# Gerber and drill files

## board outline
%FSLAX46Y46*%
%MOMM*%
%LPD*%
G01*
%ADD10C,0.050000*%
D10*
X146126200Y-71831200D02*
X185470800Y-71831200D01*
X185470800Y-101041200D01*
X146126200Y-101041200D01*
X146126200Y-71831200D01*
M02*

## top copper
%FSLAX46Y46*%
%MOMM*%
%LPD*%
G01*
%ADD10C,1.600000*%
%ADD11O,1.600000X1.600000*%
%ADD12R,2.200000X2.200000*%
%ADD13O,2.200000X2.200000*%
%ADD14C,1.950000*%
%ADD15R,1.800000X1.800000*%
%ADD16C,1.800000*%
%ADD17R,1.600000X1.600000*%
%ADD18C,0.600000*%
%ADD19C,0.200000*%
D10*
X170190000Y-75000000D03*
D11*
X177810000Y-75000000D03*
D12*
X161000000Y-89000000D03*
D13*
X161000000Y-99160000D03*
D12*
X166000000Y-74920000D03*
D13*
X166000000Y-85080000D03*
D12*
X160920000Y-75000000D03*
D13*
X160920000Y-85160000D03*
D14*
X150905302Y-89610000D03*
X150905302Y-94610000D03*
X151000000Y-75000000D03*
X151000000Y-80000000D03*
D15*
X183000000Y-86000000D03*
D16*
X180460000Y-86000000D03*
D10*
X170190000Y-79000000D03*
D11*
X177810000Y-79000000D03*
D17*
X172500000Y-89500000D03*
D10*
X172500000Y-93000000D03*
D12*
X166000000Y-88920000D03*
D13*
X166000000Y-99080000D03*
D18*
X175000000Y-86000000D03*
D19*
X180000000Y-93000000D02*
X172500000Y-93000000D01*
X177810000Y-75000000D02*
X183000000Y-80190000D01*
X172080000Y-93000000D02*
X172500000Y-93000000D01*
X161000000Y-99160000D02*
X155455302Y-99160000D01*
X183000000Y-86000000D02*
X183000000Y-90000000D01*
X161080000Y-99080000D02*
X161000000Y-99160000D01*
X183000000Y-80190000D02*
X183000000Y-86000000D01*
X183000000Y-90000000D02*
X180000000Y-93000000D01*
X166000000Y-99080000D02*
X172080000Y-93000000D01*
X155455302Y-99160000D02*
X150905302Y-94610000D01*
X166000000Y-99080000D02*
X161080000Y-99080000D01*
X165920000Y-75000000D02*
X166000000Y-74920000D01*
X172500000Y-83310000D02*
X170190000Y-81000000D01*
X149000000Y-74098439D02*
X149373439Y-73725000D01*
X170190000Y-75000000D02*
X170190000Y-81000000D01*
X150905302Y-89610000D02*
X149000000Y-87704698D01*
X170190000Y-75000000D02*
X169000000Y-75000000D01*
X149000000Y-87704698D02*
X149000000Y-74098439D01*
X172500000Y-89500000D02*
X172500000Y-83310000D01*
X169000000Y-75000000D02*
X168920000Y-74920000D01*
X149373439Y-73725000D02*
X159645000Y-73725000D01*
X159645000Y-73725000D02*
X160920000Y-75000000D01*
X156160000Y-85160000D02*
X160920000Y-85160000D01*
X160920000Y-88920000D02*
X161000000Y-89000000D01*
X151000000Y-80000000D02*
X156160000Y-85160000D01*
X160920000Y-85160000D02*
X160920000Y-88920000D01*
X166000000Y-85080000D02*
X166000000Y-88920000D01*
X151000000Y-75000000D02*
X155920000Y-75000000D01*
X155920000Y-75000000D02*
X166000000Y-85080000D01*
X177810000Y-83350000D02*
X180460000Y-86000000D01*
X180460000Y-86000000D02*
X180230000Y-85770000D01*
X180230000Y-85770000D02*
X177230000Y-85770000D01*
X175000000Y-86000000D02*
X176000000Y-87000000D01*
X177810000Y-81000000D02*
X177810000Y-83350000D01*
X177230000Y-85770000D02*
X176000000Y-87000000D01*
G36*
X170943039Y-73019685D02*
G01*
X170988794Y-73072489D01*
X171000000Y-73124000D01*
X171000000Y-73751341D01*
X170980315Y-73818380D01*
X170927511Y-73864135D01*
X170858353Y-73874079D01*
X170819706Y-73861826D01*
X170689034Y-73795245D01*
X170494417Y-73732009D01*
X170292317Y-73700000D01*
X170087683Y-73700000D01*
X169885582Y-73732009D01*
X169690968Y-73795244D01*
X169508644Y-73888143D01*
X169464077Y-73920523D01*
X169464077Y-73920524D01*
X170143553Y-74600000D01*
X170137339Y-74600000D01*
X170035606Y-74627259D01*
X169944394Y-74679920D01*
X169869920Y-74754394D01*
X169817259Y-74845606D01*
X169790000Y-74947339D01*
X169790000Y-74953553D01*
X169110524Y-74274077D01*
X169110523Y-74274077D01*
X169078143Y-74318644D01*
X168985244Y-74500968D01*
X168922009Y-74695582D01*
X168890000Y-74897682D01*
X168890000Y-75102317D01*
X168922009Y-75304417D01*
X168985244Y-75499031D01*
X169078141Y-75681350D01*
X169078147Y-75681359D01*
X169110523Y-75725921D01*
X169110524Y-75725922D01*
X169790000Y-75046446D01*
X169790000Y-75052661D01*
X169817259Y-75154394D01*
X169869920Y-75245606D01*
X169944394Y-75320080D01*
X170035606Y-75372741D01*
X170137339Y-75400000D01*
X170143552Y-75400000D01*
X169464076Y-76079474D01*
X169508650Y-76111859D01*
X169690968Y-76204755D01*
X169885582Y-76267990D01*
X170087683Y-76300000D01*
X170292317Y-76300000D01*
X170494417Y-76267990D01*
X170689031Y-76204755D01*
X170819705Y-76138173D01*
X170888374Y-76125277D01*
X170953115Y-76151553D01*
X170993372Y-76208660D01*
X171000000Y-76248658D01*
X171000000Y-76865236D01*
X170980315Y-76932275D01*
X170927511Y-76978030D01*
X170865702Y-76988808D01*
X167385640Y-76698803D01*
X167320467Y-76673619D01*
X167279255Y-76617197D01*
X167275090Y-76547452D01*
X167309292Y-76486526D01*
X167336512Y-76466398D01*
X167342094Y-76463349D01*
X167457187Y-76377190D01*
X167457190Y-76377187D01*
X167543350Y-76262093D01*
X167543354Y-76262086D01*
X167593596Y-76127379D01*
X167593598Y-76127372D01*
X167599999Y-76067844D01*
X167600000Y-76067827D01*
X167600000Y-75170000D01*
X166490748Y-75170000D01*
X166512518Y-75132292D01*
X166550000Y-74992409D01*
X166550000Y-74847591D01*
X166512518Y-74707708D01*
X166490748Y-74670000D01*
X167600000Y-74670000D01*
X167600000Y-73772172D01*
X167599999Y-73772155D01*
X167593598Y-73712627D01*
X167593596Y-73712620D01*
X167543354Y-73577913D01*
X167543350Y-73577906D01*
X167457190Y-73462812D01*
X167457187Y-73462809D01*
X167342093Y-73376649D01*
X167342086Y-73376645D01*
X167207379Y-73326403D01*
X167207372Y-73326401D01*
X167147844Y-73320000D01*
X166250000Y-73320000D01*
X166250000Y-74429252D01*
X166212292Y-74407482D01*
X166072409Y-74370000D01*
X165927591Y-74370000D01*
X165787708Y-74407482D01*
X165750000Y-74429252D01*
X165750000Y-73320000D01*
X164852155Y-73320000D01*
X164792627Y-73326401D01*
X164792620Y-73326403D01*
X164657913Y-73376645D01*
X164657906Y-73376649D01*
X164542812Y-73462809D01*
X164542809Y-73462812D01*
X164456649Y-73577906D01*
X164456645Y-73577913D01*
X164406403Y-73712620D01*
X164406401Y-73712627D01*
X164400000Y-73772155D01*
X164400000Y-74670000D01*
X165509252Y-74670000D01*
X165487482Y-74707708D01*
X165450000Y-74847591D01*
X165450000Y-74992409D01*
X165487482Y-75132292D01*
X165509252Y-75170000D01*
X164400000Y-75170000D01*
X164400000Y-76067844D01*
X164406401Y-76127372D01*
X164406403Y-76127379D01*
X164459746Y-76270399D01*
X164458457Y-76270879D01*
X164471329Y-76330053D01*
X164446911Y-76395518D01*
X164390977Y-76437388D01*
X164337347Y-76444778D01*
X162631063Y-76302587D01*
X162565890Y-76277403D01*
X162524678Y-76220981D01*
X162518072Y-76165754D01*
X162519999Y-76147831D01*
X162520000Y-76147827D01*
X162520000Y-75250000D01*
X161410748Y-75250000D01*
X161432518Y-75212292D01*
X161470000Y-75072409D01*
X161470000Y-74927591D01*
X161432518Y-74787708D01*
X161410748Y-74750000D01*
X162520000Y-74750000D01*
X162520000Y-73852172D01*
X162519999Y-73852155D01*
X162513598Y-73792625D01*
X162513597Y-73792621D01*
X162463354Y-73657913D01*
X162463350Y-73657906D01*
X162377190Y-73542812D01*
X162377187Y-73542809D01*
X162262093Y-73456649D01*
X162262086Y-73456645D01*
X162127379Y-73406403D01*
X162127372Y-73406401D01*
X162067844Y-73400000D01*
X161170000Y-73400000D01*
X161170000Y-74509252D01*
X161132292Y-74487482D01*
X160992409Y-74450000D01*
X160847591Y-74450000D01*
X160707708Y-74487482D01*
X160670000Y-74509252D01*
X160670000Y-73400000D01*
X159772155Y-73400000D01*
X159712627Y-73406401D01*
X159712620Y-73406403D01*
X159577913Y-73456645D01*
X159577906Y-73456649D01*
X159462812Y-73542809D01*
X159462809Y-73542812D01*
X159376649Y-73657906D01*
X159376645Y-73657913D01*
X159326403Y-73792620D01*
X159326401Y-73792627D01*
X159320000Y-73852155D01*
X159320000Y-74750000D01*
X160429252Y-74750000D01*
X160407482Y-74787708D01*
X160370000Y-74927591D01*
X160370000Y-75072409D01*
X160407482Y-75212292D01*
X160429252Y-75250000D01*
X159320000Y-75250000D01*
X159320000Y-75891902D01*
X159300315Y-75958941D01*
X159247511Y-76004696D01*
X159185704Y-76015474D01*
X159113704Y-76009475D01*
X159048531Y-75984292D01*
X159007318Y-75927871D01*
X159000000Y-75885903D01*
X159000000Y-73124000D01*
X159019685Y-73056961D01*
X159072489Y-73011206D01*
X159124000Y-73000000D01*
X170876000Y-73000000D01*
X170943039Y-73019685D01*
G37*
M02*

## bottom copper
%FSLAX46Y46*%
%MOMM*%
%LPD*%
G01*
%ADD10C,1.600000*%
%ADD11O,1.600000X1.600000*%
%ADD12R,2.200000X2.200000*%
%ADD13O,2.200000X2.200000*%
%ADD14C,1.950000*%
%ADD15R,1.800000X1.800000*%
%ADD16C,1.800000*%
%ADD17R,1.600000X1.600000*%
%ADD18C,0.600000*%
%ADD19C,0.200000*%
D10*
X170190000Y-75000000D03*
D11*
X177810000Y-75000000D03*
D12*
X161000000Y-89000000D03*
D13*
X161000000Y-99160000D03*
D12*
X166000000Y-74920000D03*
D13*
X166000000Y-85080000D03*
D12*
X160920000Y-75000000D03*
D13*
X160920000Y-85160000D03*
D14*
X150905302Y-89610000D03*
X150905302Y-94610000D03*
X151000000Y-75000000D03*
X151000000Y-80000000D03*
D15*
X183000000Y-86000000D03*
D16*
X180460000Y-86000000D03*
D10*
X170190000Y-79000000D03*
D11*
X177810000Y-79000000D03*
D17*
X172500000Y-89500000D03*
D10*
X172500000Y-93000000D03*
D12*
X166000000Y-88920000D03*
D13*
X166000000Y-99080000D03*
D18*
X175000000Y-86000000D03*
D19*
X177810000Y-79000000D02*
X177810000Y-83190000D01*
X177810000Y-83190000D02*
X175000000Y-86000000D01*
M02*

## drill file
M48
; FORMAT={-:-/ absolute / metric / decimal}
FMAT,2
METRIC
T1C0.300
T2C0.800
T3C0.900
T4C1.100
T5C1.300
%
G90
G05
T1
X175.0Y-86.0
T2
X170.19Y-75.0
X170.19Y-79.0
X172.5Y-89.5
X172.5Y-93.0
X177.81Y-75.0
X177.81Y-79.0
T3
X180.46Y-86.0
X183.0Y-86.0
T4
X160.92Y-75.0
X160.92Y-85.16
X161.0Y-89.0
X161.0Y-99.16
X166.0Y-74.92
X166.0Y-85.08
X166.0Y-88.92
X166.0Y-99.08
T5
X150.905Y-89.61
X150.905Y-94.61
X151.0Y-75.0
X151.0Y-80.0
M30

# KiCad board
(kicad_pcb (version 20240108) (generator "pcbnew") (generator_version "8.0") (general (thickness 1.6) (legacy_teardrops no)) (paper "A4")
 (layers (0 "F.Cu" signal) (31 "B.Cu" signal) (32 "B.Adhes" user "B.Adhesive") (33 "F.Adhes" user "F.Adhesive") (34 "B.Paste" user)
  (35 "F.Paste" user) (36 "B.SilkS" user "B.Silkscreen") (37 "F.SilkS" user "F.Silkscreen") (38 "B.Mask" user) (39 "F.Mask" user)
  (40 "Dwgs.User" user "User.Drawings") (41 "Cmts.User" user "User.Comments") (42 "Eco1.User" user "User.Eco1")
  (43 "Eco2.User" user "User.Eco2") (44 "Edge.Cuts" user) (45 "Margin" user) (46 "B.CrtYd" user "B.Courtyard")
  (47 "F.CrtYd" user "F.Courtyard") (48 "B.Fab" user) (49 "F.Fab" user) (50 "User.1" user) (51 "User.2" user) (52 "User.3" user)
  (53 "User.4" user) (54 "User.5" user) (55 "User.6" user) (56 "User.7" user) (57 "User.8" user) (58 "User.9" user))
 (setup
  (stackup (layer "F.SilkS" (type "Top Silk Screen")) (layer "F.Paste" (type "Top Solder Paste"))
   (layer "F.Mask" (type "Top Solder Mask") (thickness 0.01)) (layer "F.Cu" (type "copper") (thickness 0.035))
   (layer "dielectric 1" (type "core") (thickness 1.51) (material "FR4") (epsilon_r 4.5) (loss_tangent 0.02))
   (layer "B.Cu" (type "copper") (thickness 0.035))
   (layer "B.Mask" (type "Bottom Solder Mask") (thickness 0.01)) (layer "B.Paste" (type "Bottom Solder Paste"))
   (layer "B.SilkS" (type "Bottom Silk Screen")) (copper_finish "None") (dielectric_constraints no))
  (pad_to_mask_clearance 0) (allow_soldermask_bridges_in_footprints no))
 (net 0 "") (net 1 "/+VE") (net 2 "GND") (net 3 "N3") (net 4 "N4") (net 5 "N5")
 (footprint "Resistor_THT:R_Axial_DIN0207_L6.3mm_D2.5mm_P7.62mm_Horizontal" (layer "F.Cu") (at 170.19 75)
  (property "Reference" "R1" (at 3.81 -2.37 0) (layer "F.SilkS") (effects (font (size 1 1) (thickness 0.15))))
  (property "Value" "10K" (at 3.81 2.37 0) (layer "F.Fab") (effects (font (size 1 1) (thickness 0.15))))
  (pad "1" thru_hole circle (at 0 0) (size 1.6 1.6) (drill 0.8) (layers "*.Cu" "*.Mask") (remove_unused_layers no) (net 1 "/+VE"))
  (pad "2" thru_hole oval (at 7.62 0) (size 1.6 1.6) (drill 0.8) (layers "*.Cu" "*.Mask") (remove_unused_layers no) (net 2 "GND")))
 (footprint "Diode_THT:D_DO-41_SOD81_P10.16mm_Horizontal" (layer "F.Cu") (at 161 89 -90)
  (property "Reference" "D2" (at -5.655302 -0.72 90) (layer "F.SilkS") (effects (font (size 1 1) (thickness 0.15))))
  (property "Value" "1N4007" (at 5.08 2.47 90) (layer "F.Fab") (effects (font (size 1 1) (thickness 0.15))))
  (pad "1" thru_hole rect (at 0 0 270) (size 2.2 2.2) (drill 1.1) (layers "*.Cu" "*.Mask") (remove_unused_layers no) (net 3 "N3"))
  (pad "2" thru_hole oval (at 10.16 0 270) (size 2.2 2.2) (drill 1.1) (layers "*.Cu" "*.Mask") (remove_unused_layers no) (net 2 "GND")))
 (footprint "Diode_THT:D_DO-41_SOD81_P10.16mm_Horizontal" (layer "F.Cu") (at 166 74.92 -90)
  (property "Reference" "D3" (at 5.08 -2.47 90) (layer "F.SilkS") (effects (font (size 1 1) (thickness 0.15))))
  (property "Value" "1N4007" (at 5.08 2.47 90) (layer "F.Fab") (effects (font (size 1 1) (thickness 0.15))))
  (pad "1" thru_hole rect (at 0 0 270) (size 2.2 2.2) (drill 1.1) (layers "*.Cu" "*.Mask") (remove_unused_layers no) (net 1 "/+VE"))
  (pad "2" thru_hole oval (at 10.16 0 270) (size 2.2 2.2) (drill 1.1) (layers "*.Cu" "*.Mask") (remove_unused_layers no) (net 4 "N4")))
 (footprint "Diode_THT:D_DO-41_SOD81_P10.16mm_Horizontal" (layer "F.Cu") (at 160.92 75 -90)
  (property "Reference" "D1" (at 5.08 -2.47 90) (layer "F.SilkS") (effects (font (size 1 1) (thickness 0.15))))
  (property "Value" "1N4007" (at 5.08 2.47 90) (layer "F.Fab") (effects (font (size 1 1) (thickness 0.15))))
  (pad "1" thru_hole rect (at 0 0 270) (size 2.2 2.2) (drill 1.1) (layers "*.Cu" "*.Mask") (remove_unused_layers no) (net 1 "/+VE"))
  (pad "2" thru_hole oval (at 10.16 0 270) (size 2.2 2.2) (drill 1.1) (layers "*.Cu" "*.Mask") (remove_unused_layers no) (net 3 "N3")))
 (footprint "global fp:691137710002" (layer "F.Cu") (at 150.905302 92.11 -90)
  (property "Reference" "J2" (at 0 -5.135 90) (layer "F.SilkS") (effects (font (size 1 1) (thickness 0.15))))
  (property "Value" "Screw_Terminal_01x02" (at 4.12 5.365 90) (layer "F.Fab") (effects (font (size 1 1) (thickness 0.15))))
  (pad "1" thru_hole circle (at -2.5 0 270) (size 1.95 1.95) (drill 1.3) (layers "*.Cu" "*.Mask") (remove_unused_layers no) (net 1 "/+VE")
   (solder_mask_margin 0.102))
  (pad "2" thru_hole circle (at 2.5 0 270) (size 1.95 1.95) (drill 1.3) (layers "*.Cu" "*.Mask") (remove_unused_layers no) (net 2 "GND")
   (solder_mask_margin 0.102)))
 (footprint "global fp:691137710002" (layer "F.Cu") (at 151 77.5 -90)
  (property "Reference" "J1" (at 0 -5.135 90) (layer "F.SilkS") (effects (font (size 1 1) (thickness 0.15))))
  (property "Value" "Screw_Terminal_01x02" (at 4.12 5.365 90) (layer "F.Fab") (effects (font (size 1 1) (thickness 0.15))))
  (pad "1" thru_hole circle (at -2.5 0 270) (size 1.95 1.95) (drill 1.3) (layers "*.Cu" "*.Mask") (remove_unused_layers no) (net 4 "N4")
   (solder_mask_margin 0.102))
  (pad "2" thru_hole circle (at 2.5 0 270) (size 1.95 1.95) (drill 1.3) (layers "*.Cu" "*.Mask") (remove_unused_layers no) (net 3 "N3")
   (solder_mask_margin 0.102)))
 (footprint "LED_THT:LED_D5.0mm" (layer "F.Cu") (at 183 86 180)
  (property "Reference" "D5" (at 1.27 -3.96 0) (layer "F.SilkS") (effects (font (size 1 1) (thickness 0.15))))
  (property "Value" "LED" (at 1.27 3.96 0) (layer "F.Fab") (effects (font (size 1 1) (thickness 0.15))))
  (pad "1" thru_hole rect (at 0 0 180) (size 1.8 1.8) (drill 0.9) (layers "*.Cu" "*.Mask") (remove_unused_layers no) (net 2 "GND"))
  (pad "2" thru_hole circle (at 2.54 0 180) (size 1.8 1.8) (drill 0.9) (layers "*.Cu" "*.Mask") (remove_unused_layers no) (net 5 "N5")))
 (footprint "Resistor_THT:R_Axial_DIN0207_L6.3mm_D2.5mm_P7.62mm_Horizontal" (layer "F.Cu") (at 170.19 79)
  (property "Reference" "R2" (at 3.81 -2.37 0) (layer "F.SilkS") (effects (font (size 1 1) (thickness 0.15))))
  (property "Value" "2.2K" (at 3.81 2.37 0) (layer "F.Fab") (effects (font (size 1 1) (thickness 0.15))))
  (pad "1" thru_hole circle (at 0 0) (size 1.6 1.6) (drill 0.8) (layers "*.Cu" "*.Mask") (remove_unused_layers no) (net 1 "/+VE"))
  (pad "2" thru_hole oval (at 7.62 0) (size 1.6 1.6) (drill 0.8) (layers "*.Cu" "*.Mask") (remove_unused_layers no) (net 5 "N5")))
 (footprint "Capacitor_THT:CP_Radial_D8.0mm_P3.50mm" (layer "F.Cu") (at 172.5 89.5 -90)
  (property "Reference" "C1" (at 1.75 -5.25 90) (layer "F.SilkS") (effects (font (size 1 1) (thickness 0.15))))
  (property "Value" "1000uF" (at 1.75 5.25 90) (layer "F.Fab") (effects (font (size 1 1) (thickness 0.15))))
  (pad "1" thru_hole rect (at 0 0 270) (size 1.6 1.6) (drill 0.8) (layers "*.Cu" "*.Mask") (remove_unused_layers no) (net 1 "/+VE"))
  (pad "2" thru_hole circle (at 3.5 0 270) (size 1.6 1.6) (drill 0.8) (layers "*.Cu" "*.Mask") (remove_unused_layers no) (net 2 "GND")))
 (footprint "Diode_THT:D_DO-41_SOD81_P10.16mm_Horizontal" (layer "F.Cu") (at 166 88.92 -90)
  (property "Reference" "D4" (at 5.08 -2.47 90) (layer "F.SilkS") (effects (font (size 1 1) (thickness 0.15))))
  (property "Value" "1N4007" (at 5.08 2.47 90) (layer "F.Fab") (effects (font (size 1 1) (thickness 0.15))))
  (pad "1" thru_hole rect (at 0 0 270) (size 2.2 2.2) (drill 1.1) (layers "*.Cu" "*.Mask") (remove_unused_layers no) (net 4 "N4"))
  (pad "2" thru_hole oval (at 10.16 0 270) (size 2.2 2.2) (drill 1.1) (layers "*.Cu" "*.Mask") (remove_unused_layers no) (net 2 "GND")))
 (gr_rect (start 146.1262 71.8312) (end 185.4708 101.0412) (stroke (width 0.05) (type default)) (fill none) (layer "Edge.Cuts"))
 (segment (start 180 93) (end 172.5 93) (width 0.2) (layer "F.Cu") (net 2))
 (segment (start 177.81 75) (end 183 80.19) (width 0.2) (layer "F.Cu") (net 2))
 (segment (start 172.08 93) (end 172.5 93) (width 0.2) (layer "F.Cu") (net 2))
 (segment (start 161 99.16) (end 155.455302 99.16) (width 0.2) (layer "F.Cu") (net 2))
 (segment (start 183 86) (end 183 90) (width 0.2) (layer "F.Cu") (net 2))
 (segment (start 161.08 99.08) (end 161 99.16) (width 0.2) (layer "F.Cu") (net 2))
 (segment (start 183 80.19) (end 183 86) (width 0.2) (layer "F.Cu") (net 2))
 (segment (start 183 90) (end 180 93) (width 0.2) (layer "F.Cu") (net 2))
 (segment (start 166 99.08) (end 172.08 93) (width 0.2) (layer "F.Cu") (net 2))
 (segment (start 155.455302 99.16) (end 150.905302 94.61) (width 0.2) (layer "F.Cu") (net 2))
 (segment (start 166 99.08) (end 161.08 99.08) (width 0.2) (layer "F.Cu") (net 2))
 (segment (start 165.92 75) (end 166 74.92) (width 0.2) (layer "F.Cu") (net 1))
 (segment (start 172.5 83.31) (end 170.19 81) (width 0.2) (layer "F.Cu") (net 1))
 (segment (start 149 74.098439) (end 149.373439 73.725) (width 0.2) (layer "F.Cu") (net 1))
 (segment (start 170.19 75) (end 170.19 81) (width 0.2) (layer "F.Cu") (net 1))
 (segment (start 150.905302 89.61) (end 149 87.704698) (width 0.2) (layer "F.Cu") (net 1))
 (segment (start 170.19 75) (end 169 75) (width 0.2) (layer "F.Cu") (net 1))
 (segment (start 149 87.704698) (end 149 74.098439) (width 0.2) (layer "F.Cu") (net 1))
 (segment (start 172.5 89.5) (end 172.5 83.31) (width 0.2) (layer "F.Cu") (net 1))
 (segment (start 169 75) (end 168.92 74.92) (width 0.2) (layer "F.Cu") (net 1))
 (segment (start 149.373439 73.725) (end 159.645 73.725) (width 0.2) (layer "F.Cu") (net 1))
 (segment (start 159.645 73.725) (end 160.92 75) (width 0.2) (layer "F.Cu") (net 1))
 (segment (start 156.16 85.16) (end 160.92 85.16) (width 0.2) (layer "F.Cu") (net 3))
 (segment (start 160.92 88.92) (end 161 89) (width 0.2) (layer "F.Cu") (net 3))
 (segment (start 151 80) (end 156.16 85.16) (width 0.2) (layer "F.Cu") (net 3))
 (segment (start 160.92 85.16) (end 160.92 88.92) (width 0.2) (layer "F.Cu") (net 3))
 (segment (start 166 85.08) (end 166 88.92) (width 0.2) (layer "F.Cu") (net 4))
 (segment (start 151 75) (end 155.92 75) (width 0.2) (layer "F.Cu") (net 4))
 (segment (start 155.92 75) (end 166 85.08) (width 0.2) (layer "F.Cu") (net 4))
 (segment (start 177.81 83.35) (end 180.46 86) (width 0.2) (layer "F.Cu") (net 5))
 (segment (start 180.46 86) (end 180.23 85.77) (width 0.2) (layer "F.Cu") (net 5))
 (segment (start 180.23 85.77) (end 177.23 85.77) (width 0.2) (layer "F.Cu") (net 5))
 (segment (start 175 86) (end 176 87) (width 0.2) (layer "F.Cu") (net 5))
 (segment (start 177.81 81) (end 177.81 83.35) (width 0.2) (layer "F.Cu") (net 5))
 (segment (start 177.23 85.77) (end 176 87) (width 0.2) (layer "F.Cu") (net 5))
 (via (at 175 86) (size 0.6) (drill 0.3) (layers "F.Cu" "B.Cu") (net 5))
 (segment (start 177.81 79) (end 177.81 83.19) (width 0.2) (layer "B.Cu") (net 5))
 (segment (start 177.81 83.19) (end 175 86) (width 0.2) (layer "B.Cu") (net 5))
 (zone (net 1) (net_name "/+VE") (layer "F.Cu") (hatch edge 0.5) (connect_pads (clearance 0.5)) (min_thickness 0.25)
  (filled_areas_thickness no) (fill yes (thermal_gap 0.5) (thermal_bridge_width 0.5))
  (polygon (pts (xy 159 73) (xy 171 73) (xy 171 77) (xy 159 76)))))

